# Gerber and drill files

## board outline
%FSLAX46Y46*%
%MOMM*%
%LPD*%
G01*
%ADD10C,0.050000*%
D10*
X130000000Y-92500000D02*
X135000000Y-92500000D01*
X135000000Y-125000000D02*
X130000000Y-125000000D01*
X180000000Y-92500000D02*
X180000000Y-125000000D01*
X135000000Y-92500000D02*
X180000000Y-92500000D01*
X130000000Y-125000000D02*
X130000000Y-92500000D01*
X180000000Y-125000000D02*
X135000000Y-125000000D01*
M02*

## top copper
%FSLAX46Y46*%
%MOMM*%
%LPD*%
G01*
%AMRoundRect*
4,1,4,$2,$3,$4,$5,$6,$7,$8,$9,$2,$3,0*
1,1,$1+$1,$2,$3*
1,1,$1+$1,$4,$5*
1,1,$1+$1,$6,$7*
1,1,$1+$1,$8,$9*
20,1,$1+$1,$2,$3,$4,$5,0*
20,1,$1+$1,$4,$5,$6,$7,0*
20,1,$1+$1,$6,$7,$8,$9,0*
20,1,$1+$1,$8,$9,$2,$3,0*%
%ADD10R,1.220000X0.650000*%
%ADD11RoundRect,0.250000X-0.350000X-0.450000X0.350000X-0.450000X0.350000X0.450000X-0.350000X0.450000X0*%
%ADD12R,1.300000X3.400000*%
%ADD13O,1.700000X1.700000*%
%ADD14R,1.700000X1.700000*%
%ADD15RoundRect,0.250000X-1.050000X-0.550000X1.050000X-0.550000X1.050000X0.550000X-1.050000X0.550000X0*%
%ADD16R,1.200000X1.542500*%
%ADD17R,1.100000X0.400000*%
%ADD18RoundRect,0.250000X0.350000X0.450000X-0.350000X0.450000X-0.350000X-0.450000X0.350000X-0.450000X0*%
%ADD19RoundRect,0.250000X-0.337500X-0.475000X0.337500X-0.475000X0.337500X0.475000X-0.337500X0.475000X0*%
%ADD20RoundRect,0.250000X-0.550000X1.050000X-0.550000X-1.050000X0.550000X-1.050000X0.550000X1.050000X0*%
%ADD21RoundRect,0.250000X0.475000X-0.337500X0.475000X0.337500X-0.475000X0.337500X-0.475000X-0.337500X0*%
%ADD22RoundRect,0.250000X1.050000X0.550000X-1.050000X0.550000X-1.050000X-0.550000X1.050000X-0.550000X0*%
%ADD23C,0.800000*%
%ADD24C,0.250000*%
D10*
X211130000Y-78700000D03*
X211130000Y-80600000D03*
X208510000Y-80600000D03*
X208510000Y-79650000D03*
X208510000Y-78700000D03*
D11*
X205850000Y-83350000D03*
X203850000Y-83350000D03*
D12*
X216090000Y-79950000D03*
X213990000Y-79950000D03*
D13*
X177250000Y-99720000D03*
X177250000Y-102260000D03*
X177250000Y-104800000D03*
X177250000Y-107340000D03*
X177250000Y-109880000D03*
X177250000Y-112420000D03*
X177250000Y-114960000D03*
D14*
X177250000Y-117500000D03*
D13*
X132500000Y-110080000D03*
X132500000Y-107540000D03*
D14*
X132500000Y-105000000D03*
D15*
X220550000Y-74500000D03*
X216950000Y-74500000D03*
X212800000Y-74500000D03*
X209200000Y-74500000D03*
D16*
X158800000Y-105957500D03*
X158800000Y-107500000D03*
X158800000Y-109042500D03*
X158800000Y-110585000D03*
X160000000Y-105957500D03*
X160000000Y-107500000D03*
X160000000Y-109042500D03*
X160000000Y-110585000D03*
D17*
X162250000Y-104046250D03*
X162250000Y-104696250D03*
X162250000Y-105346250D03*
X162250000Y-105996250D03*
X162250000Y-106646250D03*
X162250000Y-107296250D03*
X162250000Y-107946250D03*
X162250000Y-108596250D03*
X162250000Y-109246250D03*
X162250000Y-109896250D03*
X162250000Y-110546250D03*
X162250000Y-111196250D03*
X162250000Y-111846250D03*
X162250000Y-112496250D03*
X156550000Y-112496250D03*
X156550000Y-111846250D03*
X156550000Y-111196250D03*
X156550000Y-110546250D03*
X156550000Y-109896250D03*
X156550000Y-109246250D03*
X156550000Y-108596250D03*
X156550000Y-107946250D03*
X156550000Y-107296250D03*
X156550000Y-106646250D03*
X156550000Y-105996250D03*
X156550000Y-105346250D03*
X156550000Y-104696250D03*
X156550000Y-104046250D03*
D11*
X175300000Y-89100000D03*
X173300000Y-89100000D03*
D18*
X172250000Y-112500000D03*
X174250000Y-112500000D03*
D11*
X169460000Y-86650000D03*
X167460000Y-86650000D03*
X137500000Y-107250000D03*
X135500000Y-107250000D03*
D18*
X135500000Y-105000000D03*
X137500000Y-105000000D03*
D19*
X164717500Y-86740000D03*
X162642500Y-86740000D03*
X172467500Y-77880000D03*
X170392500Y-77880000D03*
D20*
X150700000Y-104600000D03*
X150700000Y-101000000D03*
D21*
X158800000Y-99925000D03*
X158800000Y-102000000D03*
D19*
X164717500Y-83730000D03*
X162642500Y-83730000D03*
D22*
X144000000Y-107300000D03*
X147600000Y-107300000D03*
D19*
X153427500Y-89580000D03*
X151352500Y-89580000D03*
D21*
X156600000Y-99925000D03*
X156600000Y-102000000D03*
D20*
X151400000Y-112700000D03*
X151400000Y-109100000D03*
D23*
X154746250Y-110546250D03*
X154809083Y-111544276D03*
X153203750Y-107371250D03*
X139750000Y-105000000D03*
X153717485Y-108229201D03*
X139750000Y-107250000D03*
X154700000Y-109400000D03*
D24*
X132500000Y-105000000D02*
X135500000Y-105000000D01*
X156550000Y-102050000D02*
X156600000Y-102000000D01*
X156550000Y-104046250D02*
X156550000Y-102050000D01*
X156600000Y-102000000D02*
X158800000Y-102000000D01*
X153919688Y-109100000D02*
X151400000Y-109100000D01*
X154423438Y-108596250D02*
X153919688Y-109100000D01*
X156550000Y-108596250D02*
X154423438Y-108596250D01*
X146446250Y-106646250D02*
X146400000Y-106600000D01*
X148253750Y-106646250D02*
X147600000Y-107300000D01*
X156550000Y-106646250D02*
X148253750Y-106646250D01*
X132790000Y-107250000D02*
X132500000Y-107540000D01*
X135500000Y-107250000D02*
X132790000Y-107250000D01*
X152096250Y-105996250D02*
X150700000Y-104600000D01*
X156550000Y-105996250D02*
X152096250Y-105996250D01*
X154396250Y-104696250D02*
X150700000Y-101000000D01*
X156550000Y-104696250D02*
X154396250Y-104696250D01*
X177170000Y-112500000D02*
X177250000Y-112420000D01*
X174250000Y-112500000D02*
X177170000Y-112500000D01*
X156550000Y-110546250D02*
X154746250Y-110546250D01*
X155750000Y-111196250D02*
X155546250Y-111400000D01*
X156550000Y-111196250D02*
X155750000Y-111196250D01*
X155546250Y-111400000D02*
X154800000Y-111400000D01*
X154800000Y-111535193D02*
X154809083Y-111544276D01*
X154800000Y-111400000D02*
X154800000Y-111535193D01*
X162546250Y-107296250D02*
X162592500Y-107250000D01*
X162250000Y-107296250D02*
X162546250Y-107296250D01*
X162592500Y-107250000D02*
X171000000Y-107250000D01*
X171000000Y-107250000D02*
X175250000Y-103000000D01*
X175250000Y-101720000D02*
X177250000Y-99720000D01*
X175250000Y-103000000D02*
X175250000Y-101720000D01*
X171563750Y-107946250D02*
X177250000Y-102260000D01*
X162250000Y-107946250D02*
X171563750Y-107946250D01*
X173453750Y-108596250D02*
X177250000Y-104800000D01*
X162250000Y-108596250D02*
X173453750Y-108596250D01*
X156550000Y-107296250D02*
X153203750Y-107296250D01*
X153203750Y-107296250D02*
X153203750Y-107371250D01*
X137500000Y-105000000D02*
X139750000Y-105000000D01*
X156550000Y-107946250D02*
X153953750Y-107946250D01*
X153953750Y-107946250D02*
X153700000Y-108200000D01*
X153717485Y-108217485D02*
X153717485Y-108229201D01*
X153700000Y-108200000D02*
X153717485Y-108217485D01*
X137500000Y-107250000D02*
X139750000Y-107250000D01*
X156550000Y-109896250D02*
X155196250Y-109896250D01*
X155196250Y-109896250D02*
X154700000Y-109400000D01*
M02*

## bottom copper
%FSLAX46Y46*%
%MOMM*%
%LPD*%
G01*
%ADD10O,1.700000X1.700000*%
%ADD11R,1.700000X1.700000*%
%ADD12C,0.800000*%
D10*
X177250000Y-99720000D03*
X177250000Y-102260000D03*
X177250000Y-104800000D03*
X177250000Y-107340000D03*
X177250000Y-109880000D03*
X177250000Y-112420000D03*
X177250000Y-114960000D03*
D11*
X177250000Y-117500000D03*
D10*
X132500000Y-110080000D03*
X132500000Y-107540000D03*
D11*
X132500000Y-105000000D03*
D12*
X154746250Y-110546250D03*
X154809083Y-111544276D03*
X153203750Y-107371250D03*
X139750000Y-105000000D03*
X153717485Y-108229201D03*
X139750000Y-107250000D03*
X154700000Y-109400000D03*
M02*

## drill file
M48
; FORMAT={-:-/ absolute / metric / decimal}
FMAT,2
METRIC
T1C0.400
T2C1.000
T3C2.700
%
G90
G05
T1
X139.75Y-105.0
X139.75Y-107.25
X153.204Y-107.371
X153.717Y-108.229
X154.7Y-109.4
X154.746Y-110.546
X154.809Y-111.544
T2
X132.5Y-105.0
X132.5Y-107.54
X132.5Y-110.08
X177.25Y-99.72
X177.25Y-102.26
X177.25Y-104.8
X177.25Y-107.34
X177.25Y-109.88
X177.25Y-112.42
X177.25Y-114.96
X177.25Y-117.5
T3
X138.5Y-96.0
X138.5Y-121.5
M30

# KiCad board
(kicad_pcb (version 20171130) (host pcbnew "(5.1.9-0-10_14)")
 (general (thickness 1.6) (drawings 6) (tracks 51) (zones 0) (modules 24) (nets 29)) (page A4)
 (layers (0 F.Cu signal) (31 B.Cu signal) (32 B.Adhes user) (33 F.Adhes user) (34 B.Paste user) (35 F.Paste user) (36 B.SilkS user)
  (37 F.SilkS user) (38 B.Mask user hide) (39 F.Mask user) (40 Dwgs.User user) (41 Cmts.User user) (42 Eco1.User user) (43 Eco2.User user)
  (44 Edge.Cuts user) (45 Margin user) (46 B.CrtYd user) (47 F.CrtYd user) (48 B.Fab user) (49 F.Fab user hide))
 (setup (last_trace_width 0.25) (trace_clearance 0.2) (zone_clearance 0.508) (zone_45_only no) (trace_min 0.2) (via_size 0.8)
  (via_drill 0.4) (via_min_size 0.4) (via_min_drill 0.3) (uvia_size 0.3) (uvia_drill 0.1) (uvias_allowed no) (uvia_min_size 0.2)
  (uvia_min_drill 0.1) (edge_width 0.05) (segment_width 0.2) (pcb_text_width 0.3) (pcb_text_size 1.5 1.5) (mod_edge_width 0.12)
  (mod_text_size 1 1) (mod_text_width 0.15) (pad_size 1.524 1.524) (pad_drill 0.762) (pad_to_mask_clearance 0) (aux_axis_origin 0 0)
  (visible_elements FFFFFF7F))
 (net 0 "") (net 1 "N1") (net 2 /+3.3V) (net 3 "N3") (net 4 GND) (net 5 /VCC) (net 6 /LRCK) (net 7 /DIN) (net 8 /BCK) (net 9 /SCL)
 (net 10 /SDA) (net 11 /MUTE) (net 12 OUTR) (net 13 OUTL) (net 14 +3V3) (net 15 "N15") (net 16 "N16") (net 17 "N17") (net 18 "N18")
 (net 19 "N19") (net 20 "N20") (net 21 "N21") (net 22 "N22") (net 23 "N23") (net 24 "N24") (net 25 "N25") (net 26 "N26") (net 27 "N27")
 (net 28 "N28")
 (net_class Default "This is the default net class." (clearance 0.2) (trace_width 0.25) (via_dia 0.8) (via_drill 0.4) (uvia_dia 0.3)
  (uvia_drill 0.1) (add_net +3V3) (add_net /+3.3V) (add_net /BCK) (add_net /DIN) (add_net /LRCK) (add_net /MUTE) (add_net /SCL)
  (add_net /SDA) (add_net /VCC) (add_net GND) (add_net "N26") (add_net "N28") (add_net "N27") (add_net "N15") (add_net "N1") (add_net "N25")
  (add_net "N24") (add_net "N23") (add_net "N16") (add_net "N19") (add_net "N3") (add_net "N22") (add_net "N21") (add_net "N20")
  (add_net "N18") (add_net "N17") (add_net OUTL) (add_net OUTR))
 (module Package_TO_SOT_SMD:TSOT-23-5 (layer F.Cu) (at 209.82 79.65)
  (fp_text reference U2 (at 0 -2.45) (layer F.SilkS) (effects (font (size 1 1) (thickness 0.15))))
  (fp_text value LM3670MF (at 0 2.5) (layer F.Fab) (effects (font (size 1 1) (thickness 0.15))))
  (pad 5 smd rect (at 1.31 -0.95) (size 1.22 0.65) (layers F.Cu F.Paste F.Mask) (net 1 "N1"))
  (pad 4 smd rect (at 1.31 0.95) (size 1.22 0.65) (layers F.Cu F.Paste F.Mask) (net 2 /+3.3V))
  (pad 3 smd rect (at -1.31 0.95) (size 1.22 0.65) (layers F.Cu F.Paste F.Mask) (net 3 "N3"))
  (pad 2 smd rect (at -1.31 0) (size 1.22 0.65) (layers F.Cu F.Paste F.Mask) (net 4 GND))
  (pad 1 smd rect (at -1.31 -0.95) (size 1.22 0.65) (layers F.Cu F.Paste F.Mask) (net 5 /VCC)))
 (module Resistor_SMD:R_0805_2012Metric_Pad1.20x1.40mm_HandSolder (layer F.Cu) (at 204.85 83.35)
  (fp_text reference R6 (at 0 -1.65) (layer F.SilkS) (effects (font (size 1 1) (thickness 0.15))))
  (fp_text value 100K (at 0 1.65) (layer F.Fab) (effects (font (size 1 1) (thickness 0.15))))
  (pad 2 smd roundrect (at 1 0) (size 1.2 1.4) (layers F.Cu F.Paste F.Mask) (roundrect_rratio 0.208333) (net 5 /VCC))
  (pad 1 smd roundrect (at -1 0) (size 1.2 1.4) (layers F.Cu F.Paste F.Mask) (roundrect_rratio 0.208333) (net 3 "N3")))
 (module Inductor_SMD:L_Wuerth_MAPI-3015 (layer F.Cu) (at 215.04 79.95)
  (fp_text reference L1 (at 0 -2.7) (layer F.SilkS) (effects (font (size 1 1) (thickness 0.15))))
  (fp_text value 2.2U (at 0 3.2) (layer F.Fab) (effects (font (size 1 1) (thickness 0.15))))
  (pad 2 smd rect (at 1.05 0) (size 1.3 3.4) (layers F.Cu F.Paste F.Mask) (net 2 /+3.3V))
  (pad 1 smd rect (at -1.05 0) (size 1.3 3.4) (layers F.Cu F.Paste F.Mask) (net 1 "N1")))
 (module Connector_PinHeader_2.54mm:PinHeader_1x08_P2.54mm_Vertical (layer F.Cu) (at 177.25 117.5 180)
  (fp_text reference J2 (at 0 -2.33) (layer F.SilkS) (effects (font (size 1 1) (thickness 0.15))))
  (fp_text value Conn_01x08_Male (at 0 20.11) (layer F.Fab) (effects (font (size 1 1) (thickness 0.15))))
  (pad 8 thru_hole oval (at 0 17.78 180) (size 1.7 1.7) (drill 1) (layers *.Cu *.Mask) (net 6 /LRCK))
  (pad 7 thru_hole oval (at 0 15.24 180) (size 1.7 1.7) (drill 1) (layers *.Cu *.Mask) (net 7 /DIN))
  (pad 6 thru_hole oval (at 0 12.7 180) (size 1.7 1.7) (drill 1) (layers *.Cu *.Mask) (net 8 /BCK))
  (pad 5 thru_hole oval (at 0 10.16 180) (size 1.7 1.7) (drill 1) (layers *.Cu *.Mask) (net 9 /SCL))
  (pad 4 thru_hole oval (at 0 7.62 180) (size 1.7 1.7) (drill 1) (layers *.Cu *.Mask) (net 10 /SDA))
  (pad 3 thru_hole oval (at 0 5.08 180) (size 1.7 1.7) (drill 1) (layers *.Cu *.Mask) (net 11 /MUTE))
  (pad 2 thru_hole oval (at 0 2.54 180) (size 1.7 1.7) (drill 1) (layers *.Cu *.Mask) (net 4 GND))
  (pad 1 thru_hole rect (at 0 0 180) (size 1.7 1.7) (drill 1) (layers *.Cu *.Mask) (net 5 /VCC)))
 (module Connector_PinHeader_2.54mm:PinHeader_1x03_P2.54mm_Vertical (layer F.Cu) (at 132.5 105)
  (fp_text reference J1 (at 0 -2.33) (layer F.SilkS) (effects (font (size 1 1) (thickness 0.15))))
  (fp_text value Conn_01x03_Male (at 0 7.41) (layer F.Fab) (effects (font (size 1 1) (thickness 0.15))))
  (pad 3 thru_hole oval (at 0 5.08) (size 1.7 1.7) (drill 1) (layers *.Cu *.Mask) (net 4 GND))
  (pad 2 thru_hole oval (at 0 2.54) (size 1.7 1.7) (drill 1) (layers *.Cu *.Mask) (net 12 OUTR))
  (pad 1 thru_hole rect (at 0 0) (size 1.7 1.7) (drill 1) (layers *.Cu *.Mask) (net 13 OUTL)))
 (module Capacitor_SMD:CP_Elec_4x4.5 (layer F.Cu) (at 218.75 74.5)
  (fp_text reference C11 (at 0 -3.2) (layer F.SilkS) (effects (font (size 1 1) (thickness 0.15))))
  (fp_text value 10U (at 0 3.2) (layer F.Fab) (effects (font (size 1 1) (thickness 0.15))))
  (pad 2 smd roundrect (at 1.8 0) (size 2.6 1.6) (layers F.Cu F.Paste F.Mask) (roundrect_rratio 0.15625) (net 2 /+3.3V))
  (pad 1 smd roundrect (at -1.8 0) (size 2.6 1.6) (layers F.Cu F.Paste F.Mask) (roundrect_rratio 0.15625) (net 4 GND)))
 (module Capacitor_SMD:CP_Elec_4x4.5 (layer F.Cu) (at 211 74.5)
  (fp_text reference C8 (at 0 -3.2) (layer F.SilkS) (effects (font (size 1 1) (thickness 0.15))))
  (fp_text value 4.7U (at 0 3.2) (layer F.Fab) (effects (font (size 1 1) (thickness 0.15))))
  (pad 2 smd roundrect (at 1.8 0) (size 2.6 1.6) (layers F.Cu F.Paste F.Mask) (roundrect_rratio 0.15625) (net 4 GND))
  (pad 1 smd roundrect (at -1.8 0) (size 2.6 1.6) (layers F.Cu F.Paste F.Mask) (roundrect_rratio 0.15625) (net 5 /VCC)))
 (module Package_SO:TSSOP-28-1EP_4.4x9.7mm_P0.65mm (layer F.Cu) (at 159.4 108.27125)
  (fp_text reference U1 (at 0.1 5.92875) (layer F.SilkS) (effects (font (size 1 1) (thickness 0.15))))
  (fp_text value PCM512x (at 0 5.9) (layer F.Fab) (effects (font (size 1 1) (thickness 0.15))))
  (pad 29 smd rect (at -0.6 -2.31375) (size 1.2 1.5425) (layers F.Cu F.Paste F.Mask) (solder_paste_margin_ratio -0.2))
  (pad 29 smd rect (at -0.6 -0.77125) (size 1.2 1.5425) (layers F.Cu F.Paste F.Mask) (solder_paste_margin_ratio -0.2))
  (pad 29 smd rect (at -0.6 0.77125) (size 1.2 1.5425) (layers F.Cu F.Paste F.Mask) (solder_paste_margin_ratio -0.2))
  (pad 29 smd rect (at -0.6 2.31375) (size 1.2 1.5425) (layers F.Cu F.Paste F.Mask) (solder_paste_margin_ratio -0.2))
  (pad 29 smd rect (at 0.6 -2.31375) (size 1.2 1.5425) (layers F.Cu F.Paste F.Mask) (solder_paste_margin_ratio -0.2))
  (pad 29 smd rect (at 0.6 -0.77125) (size 1.2 1.5425) (layers F.Cu F.Paste F.Mask) (solder_paste_margin_ratio -0.2))
  (pad 29 smd rect (at 0.6 0.77125) (size 1.2 1.5425) (layers F.Cu F.Paste F.Mask) (solder_paste_margin_ratio -0.2))
  (pad 29 smd rect (at 0.6 2.31375) (size 1.2 1.5425) (layers F.Cu F.Paste F.Mask) (solder_paste_margin_ratio -0.2))
  (pad 28 smd rect (at 2.85 -4.225) (size 1.1 0.4) (layers F.Cu F.Paste F.Mask) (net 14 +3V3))
  (pad 27 smd rect (at 2.85 -3.575) (size 1.1 0.4) (layers F.Cu F.Paste F.Mask) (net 4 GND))
  (pad 26 smd rect (at 2.85 -2.925) (size 1.1 0.4) (layers F.Cu F.Paste F.Mask) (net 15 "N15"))
  (pad 25 smd rect (at 2.85 -2.275) (size 1.1 0.4) (layers F.Cu F.Paste F.Mask) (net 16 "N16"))
  (pad 24 smd rect (at 2.85 -1.625) (size 1.1 0.4) (layers F.Cu F.Paste F.Mask) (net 4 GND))
  (pad 23 smd rect (at 2.85 -0.975) (size 1.1 0.4) (layers F.Cu F.Paste F.Mask) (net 6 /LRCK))
  (pad 22 smd rect (at 2.85 -0.325) (size 1.1 0.4) (layers F.Cu F.Paste F.Mask) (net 7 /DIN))
  (pad 21 smd rect (at 2.85 0.325) (size 1.1 0.4) (layers F.Cu F.Paste F.Mask) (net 8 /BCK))
  (pad 20 smd rect (at 2.85 0.975) (size 1.1 0.4) (layers F.Cu F.Paste F.Mask) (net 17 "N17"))
  (pad 19 smd rect (at 2.85 1.625) (size 1.1 0.4) (layers F.Cu F.Paste F.Mask) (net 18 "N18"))
  (pad 18 smd rect (at 2.85 2.275) (size 1.1 0.4) (layers F.Cu F.Paste F.Mask) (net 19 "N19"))
  (pad 17 smd rect (at 2.85 2.925) (size 1.1 0.4) (layers F.Cu F.Paste F.Mask) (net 4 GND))
  (pad 16 smd rect (at 2.85 3.575) (size 1.1 0.4) (layers F.Cu F.Paste F.Mask) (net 4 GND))
  (pad 15 smd rect (at 2.85 4.225) (size 1.1 0.4) (layers F.Cu F.Paste F.Mask) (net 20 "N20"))
  (pad 14 smd rect (at -2.85 4.225) (size 1.1 0.4) (layers F.Cu F.Paste F.Mask) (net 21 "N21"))
  (pad 13 smd rect (at -2.85 3.575) (size 1.1 0.4) (layers F.Cu F.Paste F.Mask) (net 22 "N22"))
  (pad 12 smd rect (at -2.85 2.925) (size 1.1 0.4) (layers F.Cu F.Paste F.Mask) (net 9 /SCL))
  (pad 11 smd rect (at -2.85 2.275) (size 1.1 0.4) (layers F.Cu F.Paste F.Mask) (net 10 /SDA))
  (pad 10 smd rect (at -2.85 1.625) (size 1.1 0.4) (layers F.Cu F.Paste F.Mask) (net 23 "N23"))
  (pad 9 smd rect (at -2.85 0.975) (size 1.1 0.4) (layers F.Cu F.Paste F.Mask) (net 4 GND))
  (pad 8 smd rect (at -2.85 0.325) (size 1.1 0.4) (layers F.Cu F.Paste F.Mask) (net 5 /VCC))
  (pad 7 smd rect (at -2.85 -0.325) (size 1.1 0.4) (layers F.Cu F.Paste F.Mask) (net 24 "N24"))
  (pad 6 smd rect (at -2.85 -0.975) (size 1.1 0.4) (layers F.Cu F.Paste F.Mask) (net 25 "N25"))
  (pad 5 smd rect (at -2.85 -1.625) (size 1.1 0.4) (layers F.Cu F.Paste F.Mask) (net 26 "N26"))
  (pad 4 smd rect (at -2.85 -2.275) (size 1.1 0.4) (layers F.Cu F.Paste F.Mask) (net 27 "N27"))
  (pad 3 smd rect (at -2.85 -2.925) (size 1.1 0.4) (layers F.Cu F.Paste F.Mask) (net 4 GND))
  (pad 2 smd rect (at -2.85 -3.575) (size 1.1 0.4) (layers F.Cu F.Paste F.Mask) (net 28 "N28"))
  (pad 1 smd rect (at -2.85 -4.225) (size 1.1 0.4) (layers F.Cu F.Paste F.Mask) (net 5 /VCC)))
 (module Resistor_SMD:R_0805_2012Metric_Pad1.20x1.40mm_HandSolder (layer F.Cu) (at 174.3 89.1)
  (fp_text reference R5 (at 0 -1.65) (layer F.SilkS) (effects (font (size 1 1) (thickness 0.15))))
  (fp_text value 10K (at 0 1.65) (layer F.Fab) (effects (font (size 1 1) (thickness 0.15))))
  (pad 2 smd roundrect (at 1 0) (size 1.2 1.4) (layers F.Cu F.Paste F.Mask) (roundrect_rratio 0.208333) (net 19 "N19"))
  (pad 1 smd roundrect (at -1 0) (size 1.2 1.4) (layers F.Cu F.Paste F.Mask) (roundrect_rratio 0.208333) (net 14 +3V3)))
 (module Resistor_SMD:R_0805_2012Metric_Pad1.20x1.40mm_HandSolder (layer F.Cu) (at 173.25 112.5 180)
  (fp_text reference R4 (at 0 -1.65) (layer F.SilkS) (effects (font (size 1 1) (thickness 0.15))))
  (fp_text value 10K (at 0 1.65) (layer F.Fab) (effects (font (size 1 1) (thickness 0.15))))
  (pad 2 smd roundrect (at 1 0 180) (size 1.2 1.4) (layers F.Cu F.Paste F.Mask) (roundrect_rratio 0.208333) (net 16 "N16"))
  (pad 1 smd roundrect (at -1 0 180) (size 1.2 1.4) (layers F.Cu F.Paste F.Mask) (roundrect_rratio 0.208333) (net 11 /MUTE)))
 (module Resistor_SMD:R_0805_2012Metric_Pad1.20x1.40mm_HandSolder (layer F.Cu) (at 168.46 86.65)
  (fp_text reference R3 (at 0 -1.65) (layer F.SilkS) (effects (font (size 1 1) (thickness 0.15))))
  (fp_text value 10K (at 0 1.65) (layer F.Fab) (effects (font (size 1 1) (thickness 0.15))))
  (pad 2 smd roundrect (at 1 0) (size 1.2 1.4) (layers F.Cu F.Paste F.Mask) (roundrect_rratio 0.208333) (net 4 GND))
  (pad 1 smd roundrect (at -1 0) (size 1.2 1.4) (layers F.Cu F.Paste F.Mask) (roundrect_rratio 0.208333) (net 23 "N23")))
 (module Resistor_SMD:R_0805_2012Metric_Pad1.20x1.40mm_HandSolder (layer F.Cu) (at 136.5 107.25)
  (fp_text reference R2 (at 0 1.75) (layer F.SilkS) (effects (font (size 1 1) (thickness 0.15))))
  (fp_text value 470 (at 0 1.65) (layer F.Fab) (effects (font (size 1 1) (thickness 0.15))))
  (pad 2 smd roundrect (at 1 0) (size 1.2 1.4) (layers F.Cu F.Paste F.Mask) (roundrect_rratio 0.208333) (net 24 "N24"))
  (pad 1 smd roundrect (at -1 0) (size 1.2 1.4) (layers F.Cu F.Paste F.Mask) (roundrect_rratio 0.208333) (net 12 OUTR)))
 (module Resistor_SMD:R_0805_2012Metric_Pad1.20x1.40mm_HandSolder (layer F.Cu) (at 136.5 105 180)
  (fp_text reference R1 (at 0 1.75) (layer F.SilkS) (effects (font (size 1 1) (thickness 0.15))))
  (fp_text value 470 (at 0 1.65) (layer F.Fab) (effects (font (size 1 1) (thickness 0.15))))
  (pad 2 smd roundrect (at 1 0 180) (size 1.2 1.4) (layers F.Cu F.Paste F.Mask) (roundrect_rratio 0.208333) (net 13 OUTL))
  (pad 1 smd roundrect (at -1 0 180) (size 1.2 1.4) (layers F.Cu F.Paste F.Mask) (roundrect_rratio 0.208333) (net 25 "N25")))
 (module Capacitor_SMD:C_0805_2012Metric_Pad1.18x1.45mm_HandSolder (layer F.Cu) (at 163.68 86.74)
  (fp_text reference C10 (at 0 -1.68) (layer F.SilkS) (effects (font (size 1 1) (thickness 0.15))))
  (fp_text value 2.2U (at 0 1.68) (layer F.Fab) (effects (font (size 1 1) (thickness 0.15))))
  (pad 2 smd roundrect (at 1.0375 0) (size 1.175 1.45) (layers F.Cu F.Paste F.Mask) (roundrect_rratio 0.212766) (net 14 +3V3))
  (pad 1 smd roundrect (at -1.0375 0) (size 1.175 1.45) (layers F.Cu F.Paste F.Mask) (roundrect_rratio 0.212766) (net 4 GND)))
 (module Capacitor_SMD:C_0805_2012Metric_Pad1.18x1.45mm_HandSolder (layer F.Cu) (at 171.43 77.88)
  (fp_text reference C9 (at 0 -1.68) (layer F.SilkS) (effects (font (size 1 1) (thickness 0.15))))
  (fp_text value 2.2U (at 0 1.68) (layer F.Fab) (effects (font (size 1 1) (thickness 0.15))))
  (pad 2 smd roundrect (at 1.0375 0) (size 1.175 1.45) (layers F.Cu F.Paste F.Mask) (roundrect_rratio 0.212766) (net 15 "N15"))
  (pad 1 smd roundrect (at -1.0375 0) (size 1.175 1.45) (layers F.Cu F.Paste F.Mask) (roundrect_rratio 0.212766) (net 4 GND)))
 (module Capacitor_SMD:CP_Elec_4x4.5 (layer F.Cu) (at 150.7 102.8 270)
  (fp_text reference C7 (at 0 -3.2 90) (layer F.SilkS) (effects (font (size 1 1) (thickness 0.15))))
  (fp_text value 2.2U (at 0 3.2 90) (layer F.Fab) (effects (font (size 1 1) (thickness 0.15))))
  (pad 2 smd roundrect (at 1.8 0 270) (size 2.6 1.6) (layers F.Cu F.Paste F.Mask) (roundrect_rratio 0.15625) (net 27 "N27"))
  (pad 1 smd roundrect (at -1.8 0 270) (size 2.6 1.6) (layers F.Cu F.Paste F.Mask) (roundrect_rratio 0.15625) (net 28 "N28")))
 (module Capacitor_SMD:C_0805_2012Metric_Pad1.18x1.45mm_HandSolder (layer F.Cu) (at 158.8 100.9625 90)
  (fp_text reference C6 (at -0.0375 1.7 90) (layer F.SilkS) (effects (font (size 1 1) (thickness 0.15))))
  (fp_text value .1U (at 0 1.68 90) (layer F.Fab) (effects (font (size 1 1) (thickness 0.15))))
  (pad 2 smd roundrect (at 1.0375 0 90) (size 1.175 1.45) (layers F.Cu F.Paste F.Mask) (roundrect_rratio 0.212766) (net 4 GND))
  (pad 1 smd roundrect (at -1.0375 0 90) (size 1.175 1.45) (layers F.Cu F.Paste F.Mask) (roundrect_rratio 0.212766) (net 5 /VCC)))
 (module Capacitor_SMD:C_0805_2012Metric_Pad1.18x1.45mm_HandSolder (layer F.Cu) (at 163.68 83.73)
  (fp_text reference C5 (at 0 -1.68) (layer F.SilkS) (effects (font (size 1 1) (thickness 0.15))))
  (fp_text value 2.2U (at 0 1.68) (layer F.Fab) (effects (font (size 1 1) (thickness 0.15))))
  (pad 2 smd roundrect (at 1.0375 0) (size 1.175 1.45) (layers F.Cu F.Paste F.Mask) (roundrect_rratio 0.212766) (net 4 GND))
  (pad 1 smd roundrect (at -1.0375 0) (size 1.175 1.45) (layers F.Cu F.Paste F.Mask) (roundrect_rratio 0.212766) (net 12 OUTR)))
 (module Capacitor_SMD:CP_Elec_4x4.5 (layer F.Cu) (at 145.8 107.3 180)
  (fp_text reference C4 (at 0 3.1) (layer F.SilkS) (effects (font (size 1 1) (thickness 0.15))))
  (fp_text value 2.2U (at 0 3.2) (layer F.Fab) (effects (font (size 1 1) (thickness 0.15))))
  (pad 2 smd roundrect (at 1.8 0 180) (size 2.6 1.6) (layers F.Cu F.Paste F.Mask) (roundrect_rratio 0.15625) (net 4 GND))
  (pad 1 smd roundrect (at -1.8 0 180) (size 2.6 1.6) (layers F.Cu F.Paste F.Mask) (roundrect_rratio 0.15625) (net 26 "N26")))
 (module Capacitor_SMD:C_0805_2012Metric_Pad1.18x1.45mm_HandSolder (layer F.Cu) (at 152.39 89.58)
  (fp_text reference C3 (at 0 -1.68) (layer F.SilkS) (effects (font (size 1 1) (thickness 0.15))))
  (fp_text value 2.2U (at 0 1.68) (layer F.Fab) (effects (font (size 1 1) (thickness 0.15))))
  (pad 2 smd roundrect (at 1.0375 0) (size 1.175 1.45) (layers F.Cu F.Paste F.Mask) (roundrect_rratio 0.212766) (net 4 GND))
  (pad 1 smd roundrect (at -1.0375 0) (size 1.175 1.45) (layers F.Cu F.Paste F.Mask) (roundrect_rratio 0.212766) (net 13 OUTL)))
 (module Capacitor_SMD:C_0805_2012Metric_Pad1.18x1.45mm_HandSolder (layer F.Cu) (at 156.6 100.9625 90)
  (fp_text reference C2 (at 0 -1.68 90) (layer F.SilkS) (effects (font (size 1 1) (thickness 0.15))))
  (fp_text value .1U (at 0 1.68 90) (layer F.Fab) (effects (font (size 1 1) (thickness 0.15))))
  (pad 2 smd roundrect (at 1.0375 0 90) (size 1.175 1.45) (layers F.Cu F.Paste F.Mask) (roundrect_rratio 0.212766) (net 4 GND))
  (pad 1 smd roundrect (at -1.0375 0 90) (size 1.175 1.45) (layers F.Cu F.Paste F.Mask) (roundrect_rratio 0.212766) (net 5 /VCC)))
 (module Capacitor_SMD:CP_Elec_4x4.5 (layer F.Cu) (at 151.4 110.9 270)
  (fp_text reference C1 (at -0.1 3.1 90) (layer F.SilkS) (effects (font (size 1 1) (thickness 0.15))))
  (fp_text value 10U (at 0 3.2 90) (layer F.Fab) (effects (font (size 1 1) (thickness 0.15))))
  (pad 2 smd roundrect (at 1.8 0 270) (size 2.6 1.6) (layers F.Cu F.Paste F.Mask) (roundrect_rratio 0.15625) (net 4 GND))
  (pad 1 smd roundrect (at -1.8 0 270) (size 2.6 1.6) (layers F.Cu F.Paste F.Mask) (roundrect_rratio 0.15625) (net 5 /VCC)))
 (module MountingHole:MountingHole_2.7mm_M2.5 (layer F.Cu) (at 138.5 121.5)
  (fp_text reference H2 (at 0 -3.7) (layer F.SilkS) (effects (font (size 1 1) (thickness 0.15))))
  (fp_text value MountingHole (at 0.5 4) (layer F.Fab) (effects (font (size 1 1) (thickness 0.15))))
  (pad 1 np_thru_hole circle (at 0 0) (size 2.7 2.7) (drill 2.7) (layers *.Cu *.Mask)))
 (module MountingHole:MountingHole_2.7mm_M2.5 (layer F.Cu) (at 138.5 96)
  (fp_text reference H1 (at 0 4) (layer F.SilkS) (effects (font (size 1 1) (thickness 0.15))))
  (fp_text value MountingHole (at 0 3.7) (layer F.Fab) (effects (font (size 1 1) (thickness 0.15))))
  (pad 1 np_thru_hole circle (at 0 0) (size 2.7 2.7) (drill 2.7) (layers *.Cu *.Mask)))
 (gr_line (start 130 92.5) (end 135 92.5) (layer Edge.Cuts) (width 0.05))
 (gr_line (start 135 125) (end 130 125) (layer Edge.Cuts) (width 0.05))
 (gr_line (start 180 92.5) (end 180 125) (layer Edge.Cuts) (width 0.05))
 (gr_line (start 135 92.5) (end 180 92.5) (layer Edge.Cuts) (width 0.05))
 (gr_line (start 130 125) (end 130 92.5) (layer Edge.Cuts) (width 0.05))
 (gr_line (start 180 125) (end 135 125) (layer Edge.Cuts) (width 0.05))
 (segment (start 132.5 105) (end 135.5 105) (width 0.25) (layer F.Cu) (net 13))
 (segment (start 156.55 102.05) (end 156.6 102) (width 0.25) (layer F.Cu) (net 5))
 (segment (start 156.55 104.04625) (end 156.55 102.05) (width 0.25) (layer F.Cu) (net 5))
 (segment (start 156.6 102) (end 158.8 102) (width 0.25) (layer F.Cu) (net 5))
 (segment (start 153.919688 109.1) (end 151.4 109.1) (width 0.25) (layer F.Cu) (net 5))
 (segment (start 154.423438 108.59625) (end 153.919688 109.1) (width 0.25) (layer F.Cu) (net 5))
 (segment (start 156.55 108.59625) (end 154.423438 108.59625) (width 0.25) (layer F.Cu) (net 5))
 (segment (start 146.44625 106.64625) (end 146.4 106.6) (width 0.25) (layer F.Cu) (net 26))
 (segment (start 148.25375 106.64625) (end 147.6 107.3) (width 0.25) (layer F.Cu) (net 26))
 (segment (start 156.55 106.64625) (end 148.25375 106.64625) (width 0.25) (layer F.Cu) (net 26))
 (segment (start 132.79 107.25) (end 132.5 107.54) (width 0.25) (layer F.Cu) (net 12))
 (segment (start 135.5 107.25) (end 132.79 107.25) (width 0.25) (layer F.Cu) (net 12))
 (segment (start 152.09625 105.99625) (end 150.7 104.6) (width 0.25) (layer F.Cu) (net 27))
 (segment (start 156.55 105.99625) (end 152.09625 105.99625) (width 0.25) (layer F.Cu) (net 27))
 (segment (start 154.39625 104.69625) (end 150.7 101) (width 0.25) (layer F.Cu) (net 28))
 (segment (start 156.55 104.69625) (end 154.39625 104.69625) (width 0.25) (layer F.Cu) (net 28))
 (segment (start 177.17 112.5) (end 177.25 112.42) (width 0.25) (layer F.Cu) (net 11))
 (segment (start 174.25 112.5) (end 177.17 112.5) (width 0.25) (layer F.Cu) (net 11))
 (segment (start 156.55 110.54625) (end 154.74625 110.54625) (width 0.25) (layer F.Cu) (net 10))
 (via (at 154.74625 110.54625) (size 0.8) (drill 0.4) (layers F.Cu B.Cu) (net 10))
 (segment (start 155.75 111.19625) (end 155.54625 111.4) (width 0.25) (layer F.Cu) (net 9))
 (segment (start 156.55 111.19625) (end 155.75 111.19625) (width 0.25) (layer F.Cu) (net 9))
 (segment (start 155.54625 111.4) (end 154.8 111.4) (width 0.25) (layer F.Cu) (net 9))
 (via (at 154.809083 111.544276) (size 0.8) (drill 0.4) (layers F.Cu B.Cu) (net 9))
 (segment (start 154.8 111.535193) (end 154.809083 111.544276) (width 0.25) (layer F.Cu) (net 9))
 (segment (start 154.8 111.4) (end 154.8 111.535193) (width 0.25) (layer F.Cu) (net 9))
 (segment (start 162.54625 107.29625) (end 162.5925 107.25) (width 0.25) (layer F.Cu) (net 6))
 (segment (start 162.25 107.29625) (end 162.54625 107.29625) (width 0.25) (layer F.Cu) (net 6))
 (segment (start 162.5925 107.25) (end 171 107.25) (width 0.25) (layer F.Cu) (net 6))
 (segment (start 171 107.25) (end 175.25 103) (width 0.25) (layer F.Cu) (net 6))
 (segment (start 175.25 101.72) (end 177.25 99.72) (width 0.25) (layer F.Cu) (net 6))
 (segment (start 175.25 103) (end 175.25 101.72) (width 0.25) (layer F.Cu) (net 6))
 (segment (start 171.56375 107.94625) (end 177.25 102.26) (width 0.25) (layer F.Cu) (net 7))
 (segment (start 162.25 107.94625) (end 171.56375 107.94625) (width 0.25) (layer F.Cu) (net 7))
 (segment (start 173.45375 108.59625) (end 177.25 104.8) (width 0.25) (layer F.Cu) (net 8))
 (segment (start 162.25 108.59625) (end 173.45375 108.59625) (width 0.25) (layer F.Cu) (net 8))
 (segment (start 156.55 107.29625) (end 153.20375 107.29625) (width 0.25) (layer F.Cu) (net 25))
 (via (at 153.20375 107.37125) (size 0.8) (drill 0.4) (layers F.Cu B.Cu) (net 25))
 (segment (start 153.20375 107.29625) (end 153.20375 107.37125) (width 0.25) (layer F.Cu) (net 25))
 (segment (start 137.5 105) (end 139.75 105) (width 0.25) (layer F.Cu) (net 25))
 (via (at 139.75 105) (size 0.8) (drill 0.4) (layers F.Cu B.Cu) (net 25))
 (segment (start 156.55 107.94625) (end 153.95375 107.94625) (width 0.25) (layer F.Cu) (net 24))
 (segment (start 153.95375 107.94625) (end 153.7 108.2) (width 0.25) (layer F.Cu) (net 24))
 (via (at 153.717485 108.229201) (size 0.8) (drill 0.4) (layers F.Cu B.Cu) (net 24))
 (segment (start 153.717485 108.217485) (end 153.717485 108.229201) (width 0.25) (layer F.Cu) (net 24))
 (segment (start 153.7 108.2) (end 153.717485 108.217485) (width 0.25) (layer F.Cu) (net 24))
 (segment (start 137.5 107.25) (end 139.75 107.25) (width 0.25) (layer F.Cu) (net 24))
 (via (at 139.75 107.25) (size 0.8) (drill 0.4) (layers F.Cu B.Cu) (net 24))
 (segment (start 156.55 109.89625) (end 155.19625 109.89625) (width 0.25) (layer F.Cu) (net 23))
 (segment (start 155.19625 109.89625) (end 154.7 109.4) (width 0.25) (layer F.Cu) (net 23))
 (via (at 154.7 109.4) (size 0.8) (drill 0.4) (layers F.Cu B.Cu) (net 23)))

